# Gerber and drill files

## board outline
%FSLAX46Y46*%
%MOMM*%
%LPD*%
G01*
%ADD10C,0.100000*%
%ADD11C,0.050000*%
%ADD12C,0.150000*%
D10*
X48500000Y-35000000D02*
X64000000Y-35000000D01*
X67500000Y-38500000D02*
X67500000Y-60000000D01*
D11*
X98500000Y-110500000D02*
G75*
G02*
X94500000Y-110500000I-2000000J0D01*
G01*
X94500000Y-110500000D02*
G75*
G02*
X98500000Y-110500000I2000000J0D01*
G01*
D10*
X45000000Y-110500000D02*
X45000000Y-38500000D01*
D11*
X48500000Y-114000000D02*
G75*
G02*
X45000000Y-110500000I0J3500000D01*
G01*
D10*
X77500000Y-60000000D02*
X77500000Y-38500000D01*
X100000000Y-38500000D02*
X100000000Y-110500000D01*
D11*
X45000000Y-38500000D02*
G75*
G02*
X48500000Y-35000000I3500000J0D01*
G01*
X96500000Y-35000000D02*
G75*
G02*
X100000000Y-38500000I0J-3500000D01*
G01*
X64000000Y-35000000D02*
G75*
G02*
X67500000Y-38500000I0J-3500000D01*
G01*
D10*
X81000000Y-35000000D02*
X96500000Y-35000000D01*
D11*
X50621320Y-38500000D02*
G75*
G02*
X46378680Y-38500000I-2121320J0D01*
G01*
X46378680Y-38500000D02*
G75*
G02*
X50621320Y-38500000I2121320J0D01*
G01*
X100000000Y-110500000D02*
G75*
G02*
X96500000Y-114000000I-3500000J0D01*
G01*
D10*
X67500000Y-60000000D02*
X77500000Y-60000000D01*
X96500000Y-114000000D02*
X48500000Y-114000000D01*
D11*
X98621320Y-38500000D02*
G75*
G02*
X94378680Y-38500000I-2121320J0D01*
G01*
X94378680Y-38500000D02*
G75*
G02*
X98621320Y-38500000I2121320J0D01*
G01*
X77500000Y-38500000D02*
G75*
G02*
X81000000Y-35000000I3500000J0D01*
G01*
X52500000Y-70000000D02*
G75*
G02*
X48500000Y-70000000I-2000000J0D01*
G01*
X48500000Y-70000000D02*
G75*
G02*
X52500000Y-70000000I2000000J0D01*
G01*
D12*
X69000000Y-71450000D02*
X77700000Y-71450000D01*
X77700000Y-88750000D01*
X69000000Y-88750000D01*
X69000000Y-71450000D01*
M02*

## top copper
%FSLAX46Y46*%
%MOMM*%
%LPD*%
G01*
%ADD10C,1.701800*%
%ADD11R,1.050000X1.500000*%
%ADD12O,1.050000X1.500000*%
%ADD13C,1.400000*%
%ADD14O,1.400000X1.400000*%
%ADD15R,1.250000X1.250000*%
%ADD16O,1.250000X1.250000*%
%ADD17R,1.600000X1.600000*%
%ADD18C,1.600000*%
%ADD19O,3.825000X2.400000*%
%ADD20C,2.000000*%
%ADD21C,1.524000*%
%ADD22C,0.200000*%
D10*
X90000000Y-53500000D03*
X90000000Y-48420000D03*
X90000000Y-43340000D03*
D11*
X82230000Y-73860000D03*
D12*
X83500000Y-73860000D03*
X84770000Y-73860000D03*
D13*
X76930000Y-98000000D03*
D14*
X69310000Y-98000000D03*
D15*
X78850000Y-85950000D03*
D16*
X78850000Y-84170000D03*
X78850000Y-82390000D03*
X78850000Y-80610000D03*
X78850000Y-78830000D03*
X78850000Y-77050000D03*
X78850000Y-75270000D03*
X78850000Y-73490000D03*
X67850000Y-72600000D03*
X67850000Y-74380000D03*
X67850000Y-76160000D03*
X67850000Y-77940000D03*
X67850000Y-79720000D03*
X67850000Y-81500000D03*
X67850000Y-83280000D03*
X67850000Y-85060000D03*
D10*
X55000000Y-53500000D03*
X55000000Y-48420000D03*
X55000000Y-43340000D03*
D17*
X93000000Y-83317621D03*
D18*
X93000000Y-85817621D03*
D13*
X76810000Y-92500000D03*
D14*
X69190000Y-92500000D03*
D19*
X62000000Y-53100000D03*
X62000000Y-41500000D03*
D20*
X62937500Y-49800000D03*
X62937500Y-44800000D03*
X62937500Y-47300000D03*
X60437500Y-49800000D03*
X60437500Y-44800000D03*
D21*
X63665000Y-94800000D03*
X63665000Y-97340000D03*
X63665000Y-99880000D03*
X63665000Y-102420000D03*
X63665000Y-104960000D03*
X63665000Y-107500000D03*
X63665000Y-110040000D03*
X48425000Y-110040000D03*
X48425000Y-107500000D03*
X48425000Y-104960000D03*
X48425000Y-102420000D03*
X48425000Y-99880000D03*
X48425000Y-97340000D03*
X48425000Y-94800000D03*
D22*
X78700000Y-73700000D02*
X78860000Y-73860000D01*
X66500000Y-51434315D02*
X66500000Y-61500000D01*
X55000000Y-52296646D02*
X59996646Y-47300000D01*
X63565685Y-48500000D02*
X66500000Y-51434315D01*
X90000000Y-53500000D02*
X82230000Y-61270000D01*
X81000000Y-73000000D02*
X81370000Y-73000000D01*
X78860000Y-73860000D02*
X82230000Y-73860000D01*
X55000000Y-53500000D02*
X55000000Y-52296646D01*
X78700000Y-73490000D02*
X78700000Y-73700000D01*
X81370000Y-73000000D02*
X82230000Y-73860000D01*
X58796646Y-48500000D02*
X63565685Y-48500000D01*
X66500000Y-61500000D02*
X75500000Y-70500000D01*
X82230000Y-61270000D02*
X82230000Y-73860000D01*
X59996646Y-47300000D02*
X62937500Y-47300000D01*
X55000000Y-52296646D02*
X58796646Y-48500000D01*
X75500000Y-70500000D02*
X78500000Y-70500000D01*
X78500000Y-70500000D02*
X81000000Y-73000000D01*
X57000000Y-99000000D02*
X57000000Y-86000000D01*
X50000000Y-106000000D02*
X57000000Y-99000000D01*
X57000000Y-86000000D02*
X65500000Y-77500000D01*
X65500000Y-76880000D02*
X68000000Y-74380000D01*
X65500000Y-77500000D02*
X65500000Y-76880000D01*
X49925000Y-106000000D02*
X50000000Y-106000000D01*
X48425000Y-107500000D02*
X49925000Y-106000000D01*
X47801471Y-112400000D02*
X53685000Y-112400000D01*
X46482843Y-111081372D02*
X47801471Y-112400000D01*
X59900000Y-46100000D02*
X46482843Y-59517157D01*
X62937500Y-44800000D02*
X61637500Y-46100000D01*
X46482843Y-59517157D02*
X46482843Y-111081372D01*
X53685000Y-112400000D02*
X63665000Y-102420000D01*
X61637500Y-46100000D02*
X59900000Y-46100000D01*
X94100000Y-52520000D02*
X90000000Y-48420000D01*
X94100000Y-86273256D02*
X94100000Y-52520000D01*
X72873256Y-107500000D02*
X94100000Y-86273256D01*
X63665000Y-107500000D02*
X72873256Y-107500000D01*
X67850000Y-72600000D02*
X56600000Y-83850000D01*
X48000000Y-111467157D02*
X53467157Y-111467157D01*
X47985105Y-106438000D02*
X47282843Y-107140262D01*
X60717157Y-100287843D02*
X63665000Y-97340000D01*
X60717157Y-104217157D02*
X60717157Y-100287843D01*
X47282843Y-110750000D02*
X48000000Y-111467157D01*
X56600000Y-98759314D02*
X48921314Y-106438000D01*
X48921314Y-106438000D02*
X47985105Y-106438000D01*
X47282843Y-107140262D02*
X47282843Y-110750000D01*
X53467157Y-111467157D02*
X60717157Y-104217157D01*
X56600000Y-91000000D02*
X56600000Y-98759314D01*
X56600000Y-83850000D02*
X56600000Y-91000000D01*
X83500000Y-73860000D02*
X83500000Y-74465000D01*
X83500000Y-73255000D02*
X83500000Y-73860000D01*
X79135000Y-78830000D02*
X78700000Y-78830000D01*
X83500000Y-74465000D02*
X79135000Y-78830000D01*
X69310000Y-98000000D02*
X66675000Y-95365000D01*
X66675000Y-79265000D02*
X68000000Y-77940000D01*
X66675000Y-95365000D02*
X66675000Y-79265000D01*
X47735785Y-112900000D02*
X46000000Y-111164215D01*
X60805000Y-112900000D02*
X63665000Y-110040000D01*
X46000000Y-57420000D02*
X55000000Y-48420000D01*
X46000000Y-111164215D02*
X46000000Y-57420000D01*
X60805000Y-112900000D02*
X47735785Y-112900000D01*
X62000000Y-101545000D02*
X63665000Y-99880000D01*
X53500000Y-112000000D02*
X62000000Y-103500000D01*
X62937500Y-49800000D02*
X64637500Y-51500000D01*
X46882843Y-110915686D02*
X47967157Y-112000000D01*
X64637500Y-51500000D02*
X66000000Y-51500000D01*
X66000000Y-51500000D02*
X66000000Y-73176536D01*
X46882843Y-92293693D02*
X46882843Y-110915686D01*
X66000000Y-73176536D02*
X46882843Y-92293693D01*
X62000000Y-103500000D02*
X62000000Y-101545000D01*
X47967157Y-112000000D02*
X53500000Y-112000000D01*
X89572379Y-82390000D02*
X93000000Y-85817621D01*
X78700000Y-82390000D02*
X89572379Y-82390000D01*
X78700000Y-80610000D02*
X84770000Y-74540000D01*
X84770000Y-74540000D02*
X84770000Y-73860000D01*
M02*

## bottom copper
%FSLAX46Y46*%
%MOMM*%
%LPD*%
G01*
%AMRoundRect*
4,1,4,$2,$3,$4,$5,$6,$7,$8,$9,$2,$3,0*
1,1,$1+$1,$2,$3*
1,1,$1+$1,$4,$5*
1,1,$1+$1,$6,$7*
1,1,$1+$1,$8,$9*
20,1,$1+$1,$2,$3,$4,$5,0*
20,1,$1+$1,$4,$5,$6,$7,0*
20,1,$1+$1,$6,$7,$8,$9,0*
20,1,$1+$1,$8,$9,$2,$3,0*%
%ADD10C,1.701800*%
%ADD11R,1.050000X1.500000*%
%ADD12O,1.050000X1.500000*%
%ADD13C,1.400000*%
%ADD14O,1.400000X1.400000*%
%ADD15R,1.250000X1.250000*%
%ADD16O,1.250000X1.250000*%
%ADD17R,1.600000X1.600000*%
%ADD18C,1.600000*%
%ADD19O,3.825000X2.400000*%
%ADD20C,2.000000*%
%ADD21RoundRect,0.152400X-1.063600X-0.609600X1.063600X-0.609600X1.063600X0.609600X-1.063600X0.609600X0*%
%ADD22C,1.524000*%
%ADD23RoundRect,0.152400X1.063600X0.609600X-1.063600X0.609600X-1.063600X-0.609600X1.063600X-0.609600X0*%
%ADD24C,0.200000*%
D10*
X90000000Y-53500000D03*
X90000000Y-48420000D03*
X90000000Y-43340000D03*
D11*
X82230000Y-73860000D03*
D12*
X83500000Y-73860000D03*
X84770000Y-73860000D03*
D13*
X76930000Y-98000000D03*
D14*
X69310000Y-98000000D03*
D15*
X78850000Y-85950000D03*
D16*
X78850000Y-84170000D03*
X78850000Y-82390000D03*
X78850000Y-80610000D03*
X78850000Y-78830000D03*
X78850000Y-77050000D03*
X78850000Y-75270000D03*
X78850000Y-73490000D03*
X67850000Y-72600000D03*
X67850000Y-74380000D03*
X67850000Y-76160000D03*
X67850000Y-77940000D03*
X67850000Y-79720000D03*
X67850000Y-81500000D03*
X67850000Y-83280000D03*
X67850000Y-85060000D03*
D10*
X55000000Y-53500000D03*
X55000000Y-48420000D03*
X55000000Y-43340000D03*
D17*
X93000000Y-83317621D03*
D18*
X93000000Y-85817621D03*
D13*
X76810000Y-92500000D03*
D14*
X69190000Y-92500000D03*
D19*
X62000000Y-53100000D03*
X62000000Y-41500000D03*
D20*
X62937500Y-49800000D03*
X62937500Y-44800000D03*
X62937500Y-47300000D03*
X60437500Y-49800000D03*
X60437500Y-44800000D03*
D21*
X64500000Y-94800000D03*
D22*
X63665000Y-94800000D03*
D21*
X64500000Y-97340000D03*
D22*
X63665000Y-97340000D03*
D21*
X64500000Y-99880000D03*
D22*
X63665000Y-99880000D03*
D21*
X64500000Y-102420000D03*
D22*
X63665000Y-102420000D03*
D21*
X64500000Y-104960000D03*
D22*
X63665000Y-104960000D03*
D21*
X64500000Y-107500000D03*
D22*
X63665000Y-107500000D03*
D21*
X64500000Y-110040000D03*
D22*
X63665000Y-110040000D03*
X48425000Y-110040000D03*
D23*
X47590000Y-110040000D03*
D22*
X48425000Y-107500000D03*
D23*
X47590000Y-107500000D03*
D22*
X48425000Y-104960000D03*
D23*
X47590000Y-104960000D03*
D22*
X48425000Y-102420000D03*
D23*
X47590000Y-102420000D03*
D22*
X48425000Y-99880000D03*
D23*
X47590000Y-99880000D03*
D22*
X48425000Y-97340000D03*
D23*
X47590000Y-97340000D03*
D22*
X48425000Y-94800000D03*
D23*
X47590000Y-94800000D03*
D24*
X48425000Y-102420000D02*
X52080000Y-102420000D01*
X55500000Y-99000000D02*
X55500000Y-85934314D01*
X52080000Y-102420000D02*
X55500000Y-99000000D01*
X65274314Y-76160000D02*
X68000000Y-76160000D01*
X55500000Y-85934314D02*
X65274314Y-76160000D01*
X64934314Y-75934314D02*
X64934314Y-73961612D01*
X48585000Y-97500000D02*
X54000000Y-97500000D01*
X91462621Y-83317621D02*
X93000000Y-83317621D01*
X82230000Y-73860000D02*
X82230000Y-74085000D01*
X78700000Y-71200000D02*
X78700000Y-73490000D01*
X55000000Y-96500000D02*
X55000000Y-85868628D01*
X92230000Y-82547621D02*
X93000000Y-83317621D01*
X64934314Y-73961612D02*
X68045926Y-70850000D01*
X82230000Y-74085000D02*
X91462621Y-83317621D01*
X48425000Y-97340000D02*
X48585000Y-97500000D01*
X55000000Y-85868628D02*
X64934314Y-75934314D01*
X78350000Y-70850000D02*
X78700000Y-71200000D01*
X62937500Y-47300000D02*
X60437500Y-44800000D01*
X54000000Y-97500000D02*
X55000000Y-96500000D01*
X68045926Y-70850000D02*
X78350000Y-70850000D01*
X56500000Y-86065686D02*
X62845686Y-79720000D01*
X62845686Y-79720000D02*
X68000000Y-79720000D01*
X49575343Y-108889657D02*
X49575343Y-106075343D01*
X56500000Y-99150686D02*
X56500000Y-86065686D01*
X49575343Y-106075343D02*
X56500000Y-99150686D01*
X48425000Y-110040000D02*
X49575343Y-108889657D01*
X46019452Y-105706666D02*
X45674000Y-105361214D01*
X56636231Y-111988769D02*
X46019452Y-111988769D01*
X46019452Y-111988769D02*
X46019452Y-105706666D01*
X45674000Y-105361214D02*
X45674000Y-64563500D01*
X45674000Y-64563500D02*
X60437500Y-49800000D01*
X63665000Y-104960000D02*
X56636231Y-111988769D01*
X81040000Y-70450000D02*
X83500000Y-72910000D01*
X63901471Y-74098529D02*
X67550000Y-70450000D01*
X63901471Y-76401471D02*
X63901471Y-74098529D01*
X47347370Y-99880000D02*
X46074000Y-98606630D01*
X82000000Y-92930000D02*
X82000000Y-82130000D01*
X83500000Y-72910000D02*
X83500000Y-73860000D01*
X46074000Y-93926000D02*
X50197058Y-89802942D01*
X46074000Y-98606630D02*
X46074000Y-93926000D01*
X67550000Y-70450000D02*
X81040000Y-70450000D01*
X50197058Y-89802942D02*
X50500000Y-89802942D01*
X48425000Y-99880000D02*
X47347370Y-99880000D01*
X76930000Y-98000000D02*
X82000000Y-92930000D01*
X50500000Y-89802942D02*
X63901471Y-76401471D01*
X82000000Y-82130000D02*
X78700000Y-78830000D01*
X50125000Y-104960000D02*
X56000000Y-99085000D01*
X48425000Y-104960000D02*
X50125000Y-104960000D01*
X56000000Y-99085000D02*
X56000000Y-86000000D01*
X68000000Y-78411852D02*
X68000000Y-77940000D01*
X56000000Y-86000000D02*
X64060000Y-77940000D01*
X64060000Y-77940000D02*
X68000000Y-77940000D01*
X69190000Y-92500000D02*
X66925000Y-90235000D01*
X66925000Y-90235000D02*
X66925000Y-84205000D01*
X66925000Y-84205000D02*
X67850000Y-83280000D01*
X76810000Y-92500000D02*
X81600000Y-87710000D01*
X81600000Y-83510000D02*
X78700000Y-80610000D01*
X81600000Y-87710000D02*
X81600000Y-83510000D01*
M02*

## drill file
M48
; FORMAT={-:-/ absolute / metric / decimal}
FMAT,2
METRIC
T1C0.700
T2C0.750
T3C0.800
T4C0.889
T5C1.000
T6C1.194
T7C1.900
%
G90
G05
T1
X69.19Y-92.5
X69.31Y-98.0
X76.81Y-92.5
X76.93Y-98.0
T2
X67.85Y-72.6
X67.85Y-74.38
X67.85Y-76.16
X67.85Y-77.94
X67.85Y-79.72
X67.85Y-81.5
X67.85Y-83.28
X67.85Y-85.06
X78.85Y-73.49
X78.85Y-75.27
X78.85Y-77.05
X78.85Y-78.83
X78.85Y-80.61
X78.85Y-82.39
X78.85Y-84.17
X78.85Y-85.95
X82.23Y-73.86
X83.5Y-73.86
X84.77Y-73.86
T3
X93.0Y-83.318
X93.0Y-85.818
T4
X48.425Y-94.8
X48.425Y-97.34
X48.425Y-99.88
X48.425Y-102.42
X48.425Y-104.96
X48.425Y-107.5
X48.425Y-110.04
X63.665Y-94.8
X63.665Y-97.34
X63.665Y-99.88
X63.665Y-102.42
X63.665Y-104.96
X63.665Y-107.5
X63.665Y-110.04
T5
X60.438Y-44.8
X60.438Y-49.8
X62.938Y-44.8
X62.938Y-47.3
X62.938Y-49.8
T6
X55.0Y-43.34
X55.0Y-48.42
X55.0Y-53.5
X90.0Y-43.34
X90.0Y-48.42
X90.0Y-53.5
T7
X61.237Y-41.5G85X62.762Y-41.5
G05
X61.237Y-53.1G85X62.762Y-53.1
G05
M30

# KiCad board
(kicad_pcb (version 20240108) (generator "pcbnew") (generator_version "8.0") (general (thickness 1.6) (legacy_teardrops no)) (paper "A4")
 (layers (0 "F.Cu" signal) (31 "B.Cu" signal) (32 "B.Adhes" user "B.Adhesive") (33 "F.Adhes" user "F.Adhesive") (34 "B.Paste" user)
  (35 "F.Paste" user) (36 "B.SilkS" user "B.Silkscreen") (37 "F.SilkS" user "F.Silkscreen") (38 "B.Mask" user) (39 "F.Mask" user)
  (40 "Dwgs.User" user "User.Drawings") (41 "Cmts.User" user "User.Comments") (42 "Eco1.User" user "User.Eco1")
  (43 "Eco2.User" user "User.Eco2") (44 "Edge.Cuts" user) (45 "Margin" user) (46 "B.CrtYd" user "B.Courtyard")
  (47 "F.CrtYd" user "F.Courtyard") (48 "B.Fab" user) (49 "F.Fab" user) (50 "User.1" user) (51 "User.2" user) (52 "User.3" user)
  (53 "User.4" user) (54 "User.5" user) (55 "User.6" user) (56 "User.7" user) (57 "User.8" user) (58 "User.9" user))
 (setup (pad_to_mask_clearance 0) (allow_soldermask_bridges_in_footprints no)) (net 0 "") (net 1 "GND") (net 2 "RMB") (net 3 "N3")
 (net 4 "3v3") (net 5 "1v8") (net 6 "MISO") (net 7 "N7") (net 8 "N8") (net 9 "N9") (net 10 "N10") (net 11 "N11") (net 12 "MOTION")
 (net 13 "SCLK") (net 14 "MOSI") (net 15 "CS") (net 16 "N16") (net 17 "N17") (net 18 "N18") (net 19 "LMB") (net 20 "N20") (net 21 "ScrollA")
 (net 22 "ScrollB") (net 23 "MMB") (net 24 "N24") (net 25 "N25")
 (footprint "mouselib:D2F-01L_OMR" (layer "F.Cu") (at 90 53.5 90)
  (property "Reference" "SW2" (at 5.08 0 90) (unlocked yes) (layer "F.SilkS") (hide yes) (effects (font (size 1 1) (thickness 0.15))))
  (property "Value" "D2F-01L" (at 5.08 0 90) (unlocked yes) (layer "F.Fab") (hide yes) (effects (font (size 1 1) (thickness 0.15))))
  (pad "1" thru_hole circle (at 0 0 90) (size 1.7018 1.7018) (drill 1.1938) (layers "*.Cu" "*.Mask") (remove_unused_layers no) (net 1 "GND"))
  (pad "2" thru_hole circle (at 5.08 0 90) (size 1.7018 1.7018) (drill 1.1938) (layers "*.Cu" "*.Mask") (remove_unused_layers no)
   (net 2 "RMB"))
  (pad "3" thru_hole circle (at 10.16 0 90) (size 1.7018 1.7018) (drill 1.1938) (layers "*.Cu" "*.Mask") (remove_unused_layers no)
   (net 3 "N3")))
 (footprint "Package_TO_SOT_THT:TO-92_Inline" (layer "F.Cu") (at 82.23 73.86)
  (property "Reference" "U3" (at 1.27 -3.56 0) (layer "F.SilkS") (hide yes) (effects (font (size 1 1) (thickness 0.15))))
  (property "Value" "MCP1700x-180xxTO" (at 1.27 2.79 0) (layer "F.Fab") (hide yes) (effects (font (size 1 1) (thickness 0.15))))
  (pad "1" thru_hole rect (at 0 0) (size 1.05 1.5) (drill 0.75) (layers "*.Cu" "*.Mask") (remove_unused_layers no) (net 1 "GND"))
  (pad "2" thru_hole oval (at 1.27 0) (size 1.05 1.5) (drill 0.75) (layers "*.Cu" "*.Mask") (remove_unused_layers no) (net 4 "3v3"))
  (pad "3" thru_hole oval (at 2.54 0) (size 1.05 1.5) (drill 0.75) (layers "*.Cu" "*.Mask") (remove_unused_layers no) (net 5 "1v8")))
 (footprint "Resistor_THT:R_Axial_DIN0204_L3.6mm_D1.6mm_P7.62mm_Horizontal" (layer "F.Cu") (at 76.93 98 180)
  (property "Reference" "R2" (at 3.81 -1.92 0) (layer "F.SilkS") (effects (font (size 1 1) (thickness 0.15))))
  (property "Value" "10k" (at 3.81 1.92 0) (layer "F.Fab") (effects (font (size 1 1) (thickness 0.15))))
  (pad "1" thru_hole circle (at 0 0 180) (size 1.4 1.4) (drill 0.7) (layers "*.Cu" "*.Mask") (remove_unused_layers no) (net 4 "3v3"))
  (pad "2" thru_hole oval (at 7.62 0 180) (size 1.4 1.4) (drill 0.7) (layers "*.Cu" "*.Mask") (remove_unused_layers no) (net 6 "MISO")))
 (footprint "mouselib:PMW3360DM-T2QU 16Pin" (layer "F.Cu") (at 73.35 79.782 90)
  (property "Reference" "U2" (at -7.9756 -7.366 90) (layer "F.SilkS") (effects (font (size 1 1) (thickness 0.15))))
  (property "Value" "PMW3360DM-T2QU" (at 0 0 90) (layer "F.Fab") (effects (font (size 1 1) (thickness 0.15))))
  (fp_rect (start -8.968 4.35) (end 8.332 -4.35) (stroke (width 0.15) (type solid)) (fill none) (layer "Edge.Cuts"))
  (pad "1" thru_hole rect (at -6.168 5.5 90) (size 1.25 1.25) (drill 0.75) (layers "*.Cu" "*.Mask") (remove_unused_layers no) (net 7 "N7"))
  (pad "2" thru_hole oval (at -4.388 5.5 90) (size 1.25 1.25) (drill 0.75) (layers "*.Cu" "*.Mask") (remove_unused_layers no) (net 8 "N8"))
  (pad "3" thru_hole oval (at -2.608 5.5 90) (size 1.25 1.25) (drill 0.75) (layers "*.Cu" "*.Mask") (remove_unused_layers no) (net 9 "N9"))
  (pad "4" thru_hole oval (at -0.828 5.5 90) (size 1.25 1.25) (drill 0.75) (layers "*.Cu" "*.Mask") (remove_unused_layers no) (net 5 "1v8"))
  (pad "5" thru_hole oval (at 0.952 5.5 90) (size 1.25 1.25) (drill 0.75) (layers "*.Cu" "*.Mask") (remove_unused_layers no) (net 4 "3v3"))
  (pad "6" thru_hole oval (at 2.732 5.5 90) (size 1.25 1.25) (drill 0.75) (layers "*.Cu" "*.Mask") (remove_unused_layers no) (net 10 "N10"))
  (pad "7" thru_hole oval (at 4.512 5.5 90) (size 1.25 1.25) (drill 0.75) (layers "*.Cu" "*.Mask") (remove_unused_layers no) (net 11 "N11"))
  (pad "8" thru_hole oval (at 6.292 5.5 90) (size 1.25 1.25) (drill 0.75) (layers "*.Cu" "*.Mask") (remove_unused_layers no) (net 1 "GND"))
  (pad "9" thru_hole oval (at 7.182 -5.5 90) (size 1.25 1.25) (drill 0.75) (layers "*.Cu" "*.Mask") (remove_unused_layers no)
   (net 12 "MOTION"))
  (pad "10" thru_hole oval (at 5.402 -5.5 90) (size 1.25 1.25) (drill 0.75) (layers "*.Cu" "*.Mask") (remove_unused_layers no)
   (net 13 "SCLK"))
  (pad "11" thru_hole oval (at 3.622 -5.5 90) (size 1.25 1.25) (drill 0.75) (layers "*.Cu" "*.Mask") (remove_unused_layers no)
   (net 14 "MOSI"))
  (pad "12" thru_hole oval (at 1.842 -5.5 90) (size 1.25 1.25) (drill 0.75) (layers "*.Cu" "*.Mask") (remove_unused_layers no)
   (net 6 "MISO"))
  (pad "13" thru_hole oval (at 0.062 -5.5 90) (size 1.25 1.25) (drill 0.75) (layers "*.Cu" "*.Mask") (remove_unused_layers no) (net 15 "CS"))
  (pad "14" thru_hole oval (at -1.718 -5.5 90) (size 1.25 1.25) (drill 0.75) (layers "*.Cu" "*.Mask") (remove_unused_layers no)
   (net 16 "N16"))
  (pad "15" thru_hole oval (at -3.498 -5.5 90) (size 1.25 1.25) (drill 0.75) (layers "*.Cu" "*.Mask") (remove_unused_layers no)
   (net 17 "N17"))
  (pad "16" thru_hole oval (at -5.278 -5.5 90) (size 1.25 1.25) (drill 0.75) (layers "*.Cu" "*.Mask") (remove_unused_layers no)
   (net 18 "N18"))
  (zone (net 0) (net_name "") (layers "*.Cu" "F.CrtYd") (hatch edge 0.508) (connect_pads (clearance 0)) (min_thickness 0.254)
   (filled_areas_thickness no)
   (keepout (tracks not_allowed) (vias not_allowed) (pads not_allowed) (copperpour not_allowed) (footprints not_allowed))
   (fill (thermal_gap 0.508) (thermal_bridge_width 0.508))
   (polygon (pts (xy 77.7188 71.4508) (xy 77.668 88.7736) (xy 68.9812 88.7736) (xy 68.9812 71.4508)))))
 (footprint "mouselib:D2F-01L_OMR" (layer "F.Cu") (at 55 53.5 90)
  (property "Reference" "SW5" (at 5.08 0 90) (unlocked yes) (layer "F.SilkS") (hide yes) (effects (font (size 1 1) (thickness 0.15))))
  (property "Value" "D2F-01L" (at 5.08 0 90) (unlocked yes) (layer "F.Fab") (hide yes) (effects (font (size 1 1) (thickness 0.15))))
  (pad "1" thru_hole circle (at 0 0 90) (size 1.7018 1.7018) (drill 1.1938) (layers "*.Cu" "*.Mask") (remove_unused_layers no) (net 1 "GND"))
  (pad "2" thru_hole circle (at 5.08 0 90) (size 1.7018 1.7018) (drill 1.1938) (layers "*.Cu" "*.Mask") (remove_unused_layers no)
   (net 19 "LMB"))
  (pad "3" thru_hole circle (at 10.16 0 90) (size 1.7018 1.7018) (drill 1.1938) (layers "*.Cu" "*.Mask") (remove_unused_layers no)
   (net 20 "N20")))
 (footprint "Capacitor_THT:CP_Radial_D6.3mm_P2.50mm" (layer "F.Cu") (at 93 83.317621 -90)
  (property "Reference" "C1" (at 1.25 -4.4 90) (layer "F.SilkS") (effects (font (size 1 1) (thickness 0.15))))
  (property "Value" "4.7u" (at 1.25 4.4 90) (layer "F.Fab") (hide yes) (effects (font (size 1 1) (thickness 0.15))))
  (pad "1" thru_hole rect (at 0 0 270) (size 1.6 1.6) (drill 0.8) (layers "*.Cu" "*.Mask") (remove_unused_layers no) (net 1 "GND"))
  (pad "2" thru_hole circle (at 2.5 0 270) (size 1.6 1.6) (drill 0.8) (layers "*.Cu" "*.Mask") (remove_unused_layers no) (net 9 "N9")))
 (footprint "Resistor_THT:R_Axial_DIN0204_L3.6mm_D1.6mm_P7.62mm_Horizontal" (layer "F.Cu") (at 76.81 92.5 180)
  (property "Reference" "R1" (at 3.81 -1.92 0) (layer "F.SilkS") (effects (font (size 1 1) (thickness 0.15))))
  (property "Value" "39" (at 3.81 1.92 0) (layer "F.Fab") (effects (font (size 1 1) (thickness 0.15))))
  (pad "1" thru_hole circle (at 0 0 180) (size 1.4 1.4) (drill 0.7) (layers "*.Cu" "*.Mask") (remove_unused_layers no) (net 5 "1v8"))
  (pad "2" thru_hole oval (at 7.62 0 180) (size 1.4 1.4) (drill 0.7) (layers "*.Cu" "*.Mask") (remove_unused_layers no) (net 17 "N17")))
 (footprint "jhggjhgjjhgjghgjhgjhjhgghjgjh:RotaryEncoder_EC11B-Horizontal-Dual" (layer "F.Cu") (at 61.6875 47.3 90)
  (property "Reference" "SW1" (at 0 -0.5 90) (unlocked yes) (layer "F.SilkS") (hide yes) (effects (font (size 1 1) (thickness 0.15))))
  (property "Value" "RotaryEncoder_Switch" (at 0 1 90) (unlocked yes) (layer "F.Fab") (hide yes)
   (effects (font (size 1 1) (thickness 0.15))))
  (pad "" thru_hole oval (at -5.8 0.3125 90) (size 2.4 3.825) (drill oval 1.9 3.425) (layers "*.Cu" "*.Mask") (remove_unused_layers no))
  (pad "" thru_hole oval (at 5.8 0.3125 90) (size 2.4 3.825) (drill oval 1.9 3.425) (layers "*.Cu" "*.Mask") (remove_unused_layers no))
  (pad "A" thru_hole circle (at -2.5 1.25 90) (size 2 2) (drill 1) (layers "*.Cu" "*.Mask") (remove_unused_layers no) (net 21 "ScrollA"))
  (pad "B" thru_hole circle (at 2.5 1.25 90) (size 2 2) (drill 1) (layers "*.Cu" "*.Mask") (remove_unused_layers no) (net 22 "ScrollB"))
  (pad "C" thru_hole circle (at 0 1.25 90) (size 2 2) (drill 1) (layers "*.Cu" "*.Mask") (remove_unused_layers no) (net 1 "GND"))
  (pad "S1" thru_hole circle (at -2.5 -1.25 90) (size 2 2) (drill 1) (layers "*.Cu" "*.Mask") (remove_unused_layers no) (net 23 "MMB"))
  (pad "S2" thru_hole circle (at 2.5 -1.25 90) (size 2 2) (drill 1) (layers "*.Cu" "*.Mask") (remove_unused_layers no) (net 1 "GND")))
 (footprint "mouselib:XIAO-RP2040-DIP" (layer "B.Cu") (at 56.045 102.42 180)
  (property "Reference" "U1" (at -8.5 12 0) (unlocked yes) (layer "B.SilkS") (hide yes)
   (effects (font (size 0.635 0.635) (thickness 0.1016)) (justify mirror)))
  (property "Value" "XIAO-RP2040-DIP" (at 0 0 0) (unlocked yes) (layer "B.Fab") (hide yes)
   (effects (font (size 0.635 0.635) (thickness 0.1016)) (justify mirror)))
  (pad "1" smd roundrect (at -8.455 7.62) (size 2.432 1.524) (layers "B.Cu" "B.Mask") (roundrect_rratio 0.1) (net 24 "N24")
   (thermal_bridge_angle 45))
  (pad "1" thru_hole circle (at -7.62 7.62) (size 1.524 1.524) (drill 0.889) (layers "*.Cu" "*.Mask") (remove_unused_layers no)
   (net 24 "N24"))
  (pad "2" smd roundrect (at -8.455 5.08) (size 2.432 1.524) (layers "B.Cu" "B.Mask") (roundrect_rratio 0.1) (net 12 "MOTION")
   (thermal_bridge_angle 45))
  (pad "2" thru_hole circle (at -7.62 5.08) (size 1.524 1.524) (drill 0.889) (layers "*.Cu" "*.Mask") (remove_unused_layers no)
   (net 12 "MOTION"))
  (pad "3" smd roundrect (at -8.455 2.54) (size 2.432 1.524) (layers "B.Cu" "B.Mask") (roundrect_rratio 0.1) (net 21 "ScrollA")
   (thermal_bridge_angle 45))
  (pad "3" thru_hole circle (at -7.62 2.54) (size 1.524 1.524) (drill 0.889) (layers "*.Cu" "*.Mask") (remove_unused_layers no)
   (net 21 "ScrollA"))
  (pad "4" smd roundrect (at -8.455 0) (size 2.432 1.524) (layers "B.Cu" "B.Mask") (roundrect_rratio 0.1) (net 22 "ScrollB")
   (thermal_bridge_angle 45))
  (pad "4" thru_hole circle (at -7.62 0) (size 1.524 1.524) (drill 0.889) (layers "*.Cu" "*.Mask") (remove_unused_layers no)
   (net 22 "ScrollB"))
  (pad "5" smd roundrect (at -8.455 -2.54) (size 2.432 1.524) (layers "B.Cu" "B.Mask") (roundrect_rratio 0.1) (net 23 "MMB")
   (thermal_bridge_angle 45))
  (pad "5" thru_hole circle (at -7.62 -2.54) (size 1.524 1.524) (drill 0.889) (layers "*.Cu" "*.Mask") (remove_unused_layers no)
   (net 23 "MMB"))
  (pad "6" smd roundrect (at -8.455 -5.08) (size 2.432 1.524) (layers "B.Cu" "B.Mask") (roundrect_rratio 0.1) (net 2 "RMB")
   (thermal_bridge_angle 45))
  (pad "6" thru_hole circle (at -7.62 -5.08) (size 1.524 1.524) (drill 0.889) (layers "*.Cu" "*.Mask") (remove_unused_layers no)
   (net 2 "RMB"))
  (pad "7" smd roundrect (at -8.455 -7.62) (size 2.432 1.524) (layers "B.Cu" "B.Mask") (roundrect_rratio 0.1) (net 19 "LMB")
   (thermal_bridge_angle 45))
  (pad "7" thru_hole circle (at -7.62 -7.62) (size 1.524 1.524) (drill 0.889) (layers "*.Cu" "*.Mask") (remove_unused_layers no)
   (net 19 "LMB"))
  (pad "8" thru_hole circle (at 7.62 -7.62 180) (size 1.524 1.524) (drill 0.889) (layers "*.Cu" "*.Mask") (remove_unused_layers no)
   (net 15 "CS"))
  (pad "8" smd roundrect (at 8.455 -7.62 180) (size 2.432 1.524) (layers "B.Cu" "B.Mask") (roundrect_rratio 0.1) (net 15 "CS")
   (thermal_bridge_angle 45))
  (pad "9" thru_hole circle (at 7.62 -5.08 180) (size 1.524 1.524) (drill 0.889) (layers "*.Cu" "*.Mask") (remove_unused_layers no)
   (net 13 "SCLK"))
  (pad "9" smd roundrect (at 8.455 -5.08 180) (size 2.432 1.524) (layers "B.Cu" "B.Mask") (roundrect_rratio 0.1) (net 13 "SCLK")
   (thermal_bridge_angle 45))
  (pad "10" thru_hole circle (at 7.62 -2.54 180) (size 1.524 1.524) (drill 0.889) (layers "*.Cu" "*.Mask") (remove_unused_layers no)
   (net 6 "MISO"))
  (pad "10" smd roundrect (at 8.455 -2.54 180) (size 2.432 1.524) (layers "B.Cu" "B.Mask") (roundrect_rratio 0.1) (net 6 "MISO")
   (thermal_bridge_angle 45))
  (pad "11" thru_hole circle (at 7.62 0 180) (size 1.524 1.524) (drill 0.889) (layers "*.Cu" "*.Mask") (remove_unused_layers no)
   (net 14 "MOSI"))
  (pad "11" smd roundrect (at 8.455 0 180) (size 2.432 1.524) (layers "B.Cu" "B.Mask") (roundrect_rratio 0.1) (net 14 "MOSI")
   (thermal_bridge_angle 45))
  (pad "12" thru_hole circle (at 7.62 2.54 180) (size 1.524 1.524) (drill 0.889) (layers "*.Cu" "*.Mask") (remove_unused_layers no)
   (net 4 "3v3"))
  (pad "12" smd roundrect (at 8.455 2.54 180) (size 2.432 1.524) (layers "B.Cu" "B.Mask") (roundrect_rratio 0.1) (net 4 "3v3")
   (thermal_bridge_angle 45))
  (pad "13" thru_hole circle (at 7.62 5.08 180) (size 1.524 1.524) (drill 0.889) (layers "*.Cu" "*.Mask") (remove_unused_layers no)
   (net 1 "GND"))
  (pad "13" smd roundrect (at 8.455 5.08 180) (size 2.432 1.524) (layers "B.Cu" "B.Mask") (roundrect_rratio 0.1) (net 1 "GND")
   (thermal_bridge_angle 45))
  (pad "14" thru_hole circle (at 7.62 7.62 180) (size 1.524 1.524) (drill 0.889) (layers "*.Cu" "*.Mask") (remove_unused_layers no)
   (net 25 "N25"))
  (pad "14" smd roundrect (at 8.455 7.62 180) (size 2.432 1.524) (layers "B.Cu" "B.Mask") (roundrect_rratio 0.1) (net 25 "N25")
   (thermal_bridge_angle 45)))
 (gr_line (start 48.5 35) (end 64 35) (stroke (width 0.1) (type default)) (layer "Edge.Cuts"))
 (gr_line (start 67.5 38.5) (end 67.5 60) (stroke (width 0.1) (type default)) (layer "Edge.Cuts"))
 (gr_circle (center 96.5 110.5) (end 96.5 108.5) (stroke (width 0.05) (type default)) (fill none) (layer "Edge.Cuts"))
 (gr_line (start 45 110.5) (end 45 38.5) (stroke (width 0.1) (type default)) (layer "Edge.Cuts"))
 (gr_arc (start 48.5 114) (mid 46.025126 112.974874) (end 45 110.5) (stroke (width 0.05) (type default)) (layer "Edge.Cuts"))
 (gr_line (start 77.5 60) (end 77.5 38.5) (stroke (width 0.1) (type default)) (layer "Edge.Cuts"))
 (gr_line (start 100 38.5) (end 100 110.5) (stroke (width 0.1) (type default)) (layer "Edge.Cuts"))
 (gr_arc (start 45 38.5) (mid 46.025126 36.025126) (end 48.5 35) (stroke (width 0.05) (type default)) (layer "Edge.Cuts"))
 (gr_arc (start 96.5 35) (mid 98.974874 36.025126) (end 100 38.5) (stroke (width 0.05) (type default)) (layer "Edge.Cuts"))
 (gr_arc (start 64 35) (mid 66.474874 36.025126) (end 67.5 38.5) (stroke (width 0.05) (type default)) (layer "Edge.Cuts"))
 (gr_line (start 81 35) (end 96.5 35) (stroke (width 0.1) (type default)) (layer "Edge.Cuts"))
 (gr_circle (center 48.5 38.5) (end 47 40) (stroke (width 0.05) (type default)) (fill none) (layer "Edge.Cuts"))
 (gr_arc (start 100 110.5) (mid 98.974874 112.974874) (end 96.5 114) (stroke (width 0.05) (type default)) (layer "Edge.Cuts"))
 (gr_line (start 67.5 60) (end 77.5 60) (stroke (width 0.1) (type default)) (layer "Edge.Cuts"))
 (gr_line (start 96.5 114) (end 48.5 114) (stroke (width 0.1) (type default)) (layer "Edge.Cuts"))
 (gr_circle (center 96.5 38.5) (end 98 40) (stroke (width 0.05) (type default)) (fill none) (layer "Edge.Cuts"))
 (gr_arc (start 77.5 38.5) (mid 78.525126 36.025126) (end 81 35) (stroke (width 0.05) (type default)) (layer "Edge.Cuts"))
 (gr_circle (center 50.5 70) (end 50.5 72) (stroke (width 0.05) (type default)) (fill none) (layer "Edge.Cuts"))
 (segment (start 48.425 102.42) (end 52.08 102.42) (width 0.2) (layer "B.Cu") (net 14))
 (segment (start 55.5 99) (end 55.5 85.934314) (width 0.2) (layer "B.Cu") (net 14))
 (segment (start 52.08 102.42) (end 55.5 99) (width 0.2) (layer "B.Cu") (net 14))
 (segment (start 65.274314 76.16) (end 68 76.16) (width 0.2) (layer "B.Cu") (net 14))
 (segment (start 55.5 85.934314) (end 65.274314 76.16) (width 0.2) (layer "B.Cu") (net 14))
 (segment (start 78.7 73.7) (end 78.86 73.86) (width 0.2) (layer "F.Cu") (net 1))
 (segment (start 66.5 51.434315) (end 66.5 61.5) (width 0.2) (layer "F.Cu") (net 1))
 (segment (start 55 52.296646) (end 59.996646 47.3) (width 0.2) (layer "F.Cu") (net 1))
 (segment (start 63.565685 48.5) (end 66.5 51.434315) (width 0.2) (layer "F.Cu") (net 1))
 (segment (start 90 53.5) (end 82.23 61.27) (width 0.2) (layer "F.Cu") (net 1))
 (segment (start 81 73) (end 81.37 73) (width 0.2) (layer "F.Cu") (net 1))
 (segment (start 78.86 73.86) (end 82.23 73.86) (width 0.2) (layer "F.Cu") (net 1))
 (segment (start 55 53.5) (end 55 52.296646) (width 0.2) (layer "F.Cu") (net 1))
 (segment (start 78.7 73.49) (end 78.7 73.7) (width 0.2) (layer "F.Cu") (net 1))
 (segment (start 81.37 73) (end 82.23 73.86) (width 0.2) (layer "F.Cu") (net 1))
 (segment (start 58.796646 48.5) (end 63.565685 48.5) (width 0.2) (layer "F.Cu") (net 1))
 (segment (start 66.5 61.5) (end 75.5 70.5) (width 0.2) (layer "F.Cu") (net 1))
 (segment (start 82.23 61.27) (end 82.23 73.86) (width 0.2) (layer "F.Cu") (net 1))
 (segment (start 59.996646 47.3) (end 62.9375 47.3) (width 0.2) (layer "F.Cu") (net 1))
 (segment (start 55 52.296646) (end 58.796646 48.5) (width 0.2) (layer "F.Cu") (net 1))
 (segment (start 75.5 70.5) (end 78.5 70.5) (width 0.2) (layer "F.Cu") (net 1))
 (segment (start 78.5 70.5) (end 81 73) (width 0.2) (layer "F.Cu") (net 1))
 (segment (start 64.934314 75.934314) (end 64.934314 73.961612) (width 0.2) (layer "B.Cu") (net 1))
 (segment (start 48.585 97.5) (end 54 97.5) (width 0.2) (layer "B.Cu") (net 1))
 (segment (start 91.462621 83.317621) (end 93 83.317621) (width 0.2) (layer "B.Cu") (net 1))
 (segment (start 82.23 73.86) (end 82.23 74.085) (width 0.2) (layer "B.Cu") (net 1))
 (segment (start 78.7 71.2) (end 78.7 73.49) (width 0.2) (layer "B.Cu") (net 1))
 (segment (start 55 96.5) (end 55 85.868628) (width 0.2) (layer "B.Cu") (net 1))
 (segment (start 92.23 82.547621) (end 93 83.317621) (width 0.2) (layer "B.Cu") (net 1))
 (segment (start 64.934314 73.961612) (end 68.045926 70.85) (width 0.2) (layer "B.Cu") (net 1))
 (segment (start 82.23 74.085) (end 91.462621 83.317621) (width 0.2) (layer "B.Cu") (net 1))
 (segment (start 48.425 97.34) (end 48.585 97.5) (width 0.2) (layer "B.Cu") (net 1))
 (segment (start 55 85.868628) (end 64.934314 75.934314) (width 0.2) (layer "B.Cu") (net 1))
 (segment (start 78.35 70.85) (end 78.7 71.2) (width 0.2) (layer "B.Cu") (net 1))
 (segment (start 62.9375 47.3) (end 60.4375 44.8) (width 0.2) (layer "B.Cu") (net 1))
 (segment (start 54 97.5) (end 55 96.5) (width 0.2) (layer "B.Cu") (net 1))
 (segment (start 68.045926 70.85) (end 78.35 70.85) (width 0.2) (layer "B.Cu") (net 1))
 (segment (start 56.5 86.065686) (end 62.845686 79.72) (width 0.2) (layer "B.Cu") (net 15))
 (segment (start 62.845686 79.72) (end 68 79.72) (width 0.2) (layer "B.Cu") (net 15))
 (segment (start 49.575343 108.889657) (end 49.575343 106.075343) (width 0.2) (layer "B.Cu") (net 15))
 (segment (start 56.5 99.150686) (end 56.5 86.065686) (width 0.2) (layer "B.Cu") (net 15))
 (segment (start 49.575343 106.075343) (end 56.5 99.150686) (width 0.2) (layer "B.Cu") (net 15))
 (segment (start 48.425 110.04) (end 49.575343 108.889657) (width 0.2) (layer "B.Cu") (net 15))
 (segment (start 57 99) (end 57 86) (width 0.2) (layer "F.Cu") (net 13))
 (segment (start 50 106) (end 57 99) (width 0.2) (layer "F.Cu") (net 13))
 (segment (start 57 86) (end 65.5 77.5) (width 0.2) (layer "F.Cu") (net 13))
 (segment (start 65.5 76.88) (end 68 74.38) (width 0.2) (layer "F.Cu") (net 13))
 (segment (start 65.5 77.5) (end 65.5 76.88) (width 0.2) (layer "F.Cu") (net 13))
 (segment (start 49.925 106) (end 50 106) (width 0.2) (layer "F.Cu") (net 13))
 (segment (start 48.425 107.5) (end 49.925 106) (width 0.2) (layer "F.Cu") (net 13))
 (segment (start 47.801471 112.4) (end 53.685 112.4) (width 0.2) (layer "F.Cu") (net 22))
 (segment (start 46.482843 111.081372) (end 47.801471 112.4) (width 0.2) (layer "F.Cu") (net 22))
 (segment (start 59.9 46.1) (end 46.482843 59.517157) (width 0.2) (layer "F.Cu") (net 22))
 (segment (start 62.9375 44.8) (end 61.6375 46.1) (width 0.2) (layer "F.Cu") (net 22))
 (segment (start 46.482843 59.517157) (end 46.482843 111.081372) (width 0.2) (layer "F.Cu") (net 22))
 (segment (start 53.685 112.4) (end 63.665 102.42) (width 0.2) (layer "F.Cu") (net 22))
 (segment (start 61.6375 46.1) (end 59.9 46.1) (width 0.2) (layer "F.Cu") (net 22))
 (segment (start 94.1 52.52) (end 90 48.42) (width 0.2) (layer "F.Cu") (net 2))
 (segment (start 94.1 86.273256) (end 94.1 52.52) (width 0.2) (layer "F.Cu") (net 2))
 (segment (start 72.873256 107.5) (end 94.1 86.273256) (width 0.2) (layer "F.Cu") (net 2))
 (segment (start 63.665 107.5) (end 72.873256 107.5) (width 0.2) (layer "F.Cu") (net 2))
 (segment (start 46.019452 105.706666) (end 45.674 105.361214) (width 0.2) (layer "B.Cu") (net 23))
 (segment (start 56.636231 111.988769) (end 46.019452 111.988769) (width 0.2) (layer "B.Cu") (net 23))
 (segment (start 46.019452 111.988769) (end 46.019452 105.706666) (width 0.2) (layer "B.Cu") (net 23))
 (segment (start 45.674 105.361214) (end 45.674 64.5635) (width 0.2) (layer "B.Cu") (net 23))
 (segment (start 45.674 64.5635) (end 60.4375 49.8) (width 0.2) (layer "B.Cu") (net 23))
 (segment (start 63.665 104.96) (end 56.636231 111.988769) (width 0.2) (layer "B.Cu") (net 23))
 (segment (start 67.85 72.6) (end 56.6 83.85) (width 0.2) (layer "F.Cu") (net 12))
 (segment (start 48 111.467157) (end 53.467157 111.467157) (width 0.2) (layer "F.Cu") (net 12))
 (segment (start 47.985105 106.438) (end 47.282843 107.140262) (width 0.2) (layer "F.Cu") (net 12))
 (segment (start 60.717157 100.287843) (end 63.665 97.34) (width 0.2) (layer "F.Cu") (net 12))
 (segment (start 60.717157 104.217157) (end 60.717157 100.287843) (width 0.2) (layer "F.Cu") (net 12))
 (segment (start 47.282843 110.75) (end 48 111.467157) (width 0.2) (layer "F.Cu") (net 12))
 (segment (start 56.6 98.759314) (end 48.921314 106.438) (width 0.2) (layer "F.Cu") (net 12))
 (segment (start 48.921314 106.438) (end 47.985105 106.438) (width 0.2) (layer "F.Cu") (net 12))
 (segment (start 47.282843 107.140262) (end 47.282843 110.75) (width 0.2) (layer "F.Cu") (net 12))
 (segment (start 53.467157 111.467157) (end 60.717157 104.217157) (width 0.2) (layer "F.Cu") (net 12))
 (segment (start 56.6 91) (end 56.6 98.759314) (width 0.2) (layer "F.Cu") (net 12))
 (segment (start 56.6 83.85) (end 56.6 91) (width 0.2) (layer "F.Cu") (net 12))
 (segment (start 83.5 73.86) (end 83.5 74.465) (width 0.2) (layer "F.Cu") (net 4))
 (segment (start 83.5 73.255) (end 83.5 73.86) (width 0.2) (layer "F.Cu") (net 4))
 (segment (start 79.135 78.83) (end 78.7 78.83) (width 0.2) (layer "F.Cu") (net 4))
 (segment (start 83.5 74.465) (end 79.135 78.83) (width 0.2) (layer "F.Cu") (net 4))
 (segment (start 81.04 70.45) (end 83.5 72.91) (width 0.2) (layer "B.Cu") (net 4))
 (segment (start 63.901471 74.098529) (end 67.55 70.45) (width 0.2) (layer "B.Cu") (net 4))
 (segment (start 63.901471 76.401471) (end 63.901471 74.098529) (width 0.2) (layer "B.Cu") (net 4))
 (segment (start 47.34737 99.88) (end 46.074 98.60663) (width 0.2) (layer "B.Cu") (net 4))
 (segment (start 82 92.93) (end 82 82.13) (width 0.2) (layer "B.Cu") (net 4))
 (segment (start 83.5 72.91) (end 83.5 73.86) (width 0.2) (layer "B.Cu") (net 4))
 (segment (start 46.074 93.926) (end 50.197058 89.802942) (width 0.2) (layer "B.Cu") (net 4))
 (segment (start 46.074 98.60663) (end 46.074 93.926) (width 0.2) (layer "B.Cu") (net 4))
 (segment (start 67.55 70.45) (end 81.04 70.45) (width 0.2) (layer "B.Cu") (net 4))
 (segment (start 50.197058 89.802942) (end 50.5 89.802942) (width 0.2) (layer "B.Cu") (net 4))
 (segment (start 48.425 99.88) (end 47.34737 99.88) (width 0.2) (layer "B.Cu") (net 4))
 (segment (start 76.93 98) (end 82 92.93) (width 0.2) (layer "B.Cu") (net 4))
 (segment (start 50.5 89.802942) (end 63.901471 76.401471) (width 0.2) (layer "B.Cu") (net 4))
 (segment (start 82 82.13) (end 78.7 78.83) (width 0.2) (layer "B.Cu") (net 4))
 (segment (start 69.31 98) (end 66.675 95.365) (width 0.2) (layer "F.Cu") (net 6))
 (segment (start 66.675 79.265) (end 68 77.94) (width 0.2) (layer "F.Cu") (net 6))
 (segment (start 66.675 95.365) (end 66.675 79.265) (width 0.2) (layer "F.Cu") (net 6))
 (segment (start 50.125 104.96) (end 56 99.085) (width 0.2) (layer "B.Cu") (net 6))
 (segment (start 48.425 104.96) (end 50.125 104.96) (width 0.2) (layer "B.Cu") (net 6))
 (segment (start 56 99.085) (end 56 86) (width 0.2) (layer "B.Cu") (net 6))
 (segment (start 68 78.411852) (end 68 77.94) (width 0.2) (layer "B.Cu") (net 6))
 (segment (start 56 86) (end 64.06 77.94) (width 0.2) (layer "B.Cu") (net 6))
 (segment (start 64.06 77.94) (end 68 77.94) (width 0.2) (layer "B.Cu") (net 6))
 (segment (start 47.735785 112.9) (end 46 111.164215) (width 0.2) (layer "F.Cu") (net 19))
 (segment (start 60.805 112.9) (end 63.665 110.04) (width 0.2) (layer "F.Cu") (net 19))
 (segment (start 46 57.42) (end 55 48.42) (width 0.2) (layer "F.Cu") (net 19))
 (segment (start 46 111.164215) (end 46 57.42) (width 0.2) (layer "F.Cu") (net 19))
 (segment (start 60.805 112.9) (end 47.735785 112.9) (width 0.2) (layer "F.Cu") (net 19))
 (segment (start 62 101.545) (end 63.665 99.88) (width 0.2) (layer "F.Cu") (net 21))
 (segment (start 53.5 112) (end 62 103.5) (width 0.2) (layer "F.Cu") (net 21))
 (segment (start 62.9375 49.8) (end 64.6375 51.5) (width 0.2) (layer "F.Cu") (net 21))
 (segment (start 46.882843 110.915686) (end 47.967157 112) (width 0.2) (layer "F.Cu") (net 21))
 (segment (start 64.6375 51.5) (end 66 51.5) (width 0.2) (layer "F.Cu") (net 21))
 (segment (start 66 51.5) (end 66 73.176536) (width 0.2) (layer "F.Cu") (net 21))
 (segment (start 46.882843 92.293693) (end 46.882843 110.915686) (width 0.2) (layer "F.Cu") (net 21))
 (segment (start 66 73.176536) (end 46.882843 92.293693) (width 0.2) (layer "F.Cu") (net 21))
 (segment (start 62 103.5) (end 62 101.545) (width 0.2) (layer "F.Cu") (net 21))
 (segment (start 47.967157 112) (end 53.5 112) (width 0.2) (layer "F.Cu") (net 21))
 (segment (start 69.19 92.5) (end 66.925 90.235) (width 0.2) (layer "B.Cu") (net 17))
 (segment (start 66.925 90.235) (end 66.925 84.205) (width 0.2) (layer "B.Cu") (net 17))
 (segment (start 66.925 84.205) (end 67.85 83.28) (width 0.2) (layer "B.Cu") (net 17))
 (segment (start 89.572379 82.39) (end 93 85.817621) (width 0.2) (layer "F.Cu") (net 9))
 (segment (start 78.7 82.39) (end 89.572379 82.39) (width 0.2) (layer "F.Cu") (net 9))
 (segment (start 78.7 80.61) (end 84.77 74.54) (width 0.2) (layer "F.Cu") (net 5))
 (segment (start 84.77 74.54) (end 84.77 73.86) (width 0.2) (layer "F.Cu") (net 5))
 (segment (start 76.81 92.5) (end 81.6 87.71) (width 0.2) (layer "B.Cu") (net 5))
 (segment (start 81.6 83.51) (end 78.7 80.61) (width 0.2) (layer "B.Cu") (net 5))
 (segment (start 81.6 87.71) (end 81.6 83.51) (width 0.2) (layer "B.Cu") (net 5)))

